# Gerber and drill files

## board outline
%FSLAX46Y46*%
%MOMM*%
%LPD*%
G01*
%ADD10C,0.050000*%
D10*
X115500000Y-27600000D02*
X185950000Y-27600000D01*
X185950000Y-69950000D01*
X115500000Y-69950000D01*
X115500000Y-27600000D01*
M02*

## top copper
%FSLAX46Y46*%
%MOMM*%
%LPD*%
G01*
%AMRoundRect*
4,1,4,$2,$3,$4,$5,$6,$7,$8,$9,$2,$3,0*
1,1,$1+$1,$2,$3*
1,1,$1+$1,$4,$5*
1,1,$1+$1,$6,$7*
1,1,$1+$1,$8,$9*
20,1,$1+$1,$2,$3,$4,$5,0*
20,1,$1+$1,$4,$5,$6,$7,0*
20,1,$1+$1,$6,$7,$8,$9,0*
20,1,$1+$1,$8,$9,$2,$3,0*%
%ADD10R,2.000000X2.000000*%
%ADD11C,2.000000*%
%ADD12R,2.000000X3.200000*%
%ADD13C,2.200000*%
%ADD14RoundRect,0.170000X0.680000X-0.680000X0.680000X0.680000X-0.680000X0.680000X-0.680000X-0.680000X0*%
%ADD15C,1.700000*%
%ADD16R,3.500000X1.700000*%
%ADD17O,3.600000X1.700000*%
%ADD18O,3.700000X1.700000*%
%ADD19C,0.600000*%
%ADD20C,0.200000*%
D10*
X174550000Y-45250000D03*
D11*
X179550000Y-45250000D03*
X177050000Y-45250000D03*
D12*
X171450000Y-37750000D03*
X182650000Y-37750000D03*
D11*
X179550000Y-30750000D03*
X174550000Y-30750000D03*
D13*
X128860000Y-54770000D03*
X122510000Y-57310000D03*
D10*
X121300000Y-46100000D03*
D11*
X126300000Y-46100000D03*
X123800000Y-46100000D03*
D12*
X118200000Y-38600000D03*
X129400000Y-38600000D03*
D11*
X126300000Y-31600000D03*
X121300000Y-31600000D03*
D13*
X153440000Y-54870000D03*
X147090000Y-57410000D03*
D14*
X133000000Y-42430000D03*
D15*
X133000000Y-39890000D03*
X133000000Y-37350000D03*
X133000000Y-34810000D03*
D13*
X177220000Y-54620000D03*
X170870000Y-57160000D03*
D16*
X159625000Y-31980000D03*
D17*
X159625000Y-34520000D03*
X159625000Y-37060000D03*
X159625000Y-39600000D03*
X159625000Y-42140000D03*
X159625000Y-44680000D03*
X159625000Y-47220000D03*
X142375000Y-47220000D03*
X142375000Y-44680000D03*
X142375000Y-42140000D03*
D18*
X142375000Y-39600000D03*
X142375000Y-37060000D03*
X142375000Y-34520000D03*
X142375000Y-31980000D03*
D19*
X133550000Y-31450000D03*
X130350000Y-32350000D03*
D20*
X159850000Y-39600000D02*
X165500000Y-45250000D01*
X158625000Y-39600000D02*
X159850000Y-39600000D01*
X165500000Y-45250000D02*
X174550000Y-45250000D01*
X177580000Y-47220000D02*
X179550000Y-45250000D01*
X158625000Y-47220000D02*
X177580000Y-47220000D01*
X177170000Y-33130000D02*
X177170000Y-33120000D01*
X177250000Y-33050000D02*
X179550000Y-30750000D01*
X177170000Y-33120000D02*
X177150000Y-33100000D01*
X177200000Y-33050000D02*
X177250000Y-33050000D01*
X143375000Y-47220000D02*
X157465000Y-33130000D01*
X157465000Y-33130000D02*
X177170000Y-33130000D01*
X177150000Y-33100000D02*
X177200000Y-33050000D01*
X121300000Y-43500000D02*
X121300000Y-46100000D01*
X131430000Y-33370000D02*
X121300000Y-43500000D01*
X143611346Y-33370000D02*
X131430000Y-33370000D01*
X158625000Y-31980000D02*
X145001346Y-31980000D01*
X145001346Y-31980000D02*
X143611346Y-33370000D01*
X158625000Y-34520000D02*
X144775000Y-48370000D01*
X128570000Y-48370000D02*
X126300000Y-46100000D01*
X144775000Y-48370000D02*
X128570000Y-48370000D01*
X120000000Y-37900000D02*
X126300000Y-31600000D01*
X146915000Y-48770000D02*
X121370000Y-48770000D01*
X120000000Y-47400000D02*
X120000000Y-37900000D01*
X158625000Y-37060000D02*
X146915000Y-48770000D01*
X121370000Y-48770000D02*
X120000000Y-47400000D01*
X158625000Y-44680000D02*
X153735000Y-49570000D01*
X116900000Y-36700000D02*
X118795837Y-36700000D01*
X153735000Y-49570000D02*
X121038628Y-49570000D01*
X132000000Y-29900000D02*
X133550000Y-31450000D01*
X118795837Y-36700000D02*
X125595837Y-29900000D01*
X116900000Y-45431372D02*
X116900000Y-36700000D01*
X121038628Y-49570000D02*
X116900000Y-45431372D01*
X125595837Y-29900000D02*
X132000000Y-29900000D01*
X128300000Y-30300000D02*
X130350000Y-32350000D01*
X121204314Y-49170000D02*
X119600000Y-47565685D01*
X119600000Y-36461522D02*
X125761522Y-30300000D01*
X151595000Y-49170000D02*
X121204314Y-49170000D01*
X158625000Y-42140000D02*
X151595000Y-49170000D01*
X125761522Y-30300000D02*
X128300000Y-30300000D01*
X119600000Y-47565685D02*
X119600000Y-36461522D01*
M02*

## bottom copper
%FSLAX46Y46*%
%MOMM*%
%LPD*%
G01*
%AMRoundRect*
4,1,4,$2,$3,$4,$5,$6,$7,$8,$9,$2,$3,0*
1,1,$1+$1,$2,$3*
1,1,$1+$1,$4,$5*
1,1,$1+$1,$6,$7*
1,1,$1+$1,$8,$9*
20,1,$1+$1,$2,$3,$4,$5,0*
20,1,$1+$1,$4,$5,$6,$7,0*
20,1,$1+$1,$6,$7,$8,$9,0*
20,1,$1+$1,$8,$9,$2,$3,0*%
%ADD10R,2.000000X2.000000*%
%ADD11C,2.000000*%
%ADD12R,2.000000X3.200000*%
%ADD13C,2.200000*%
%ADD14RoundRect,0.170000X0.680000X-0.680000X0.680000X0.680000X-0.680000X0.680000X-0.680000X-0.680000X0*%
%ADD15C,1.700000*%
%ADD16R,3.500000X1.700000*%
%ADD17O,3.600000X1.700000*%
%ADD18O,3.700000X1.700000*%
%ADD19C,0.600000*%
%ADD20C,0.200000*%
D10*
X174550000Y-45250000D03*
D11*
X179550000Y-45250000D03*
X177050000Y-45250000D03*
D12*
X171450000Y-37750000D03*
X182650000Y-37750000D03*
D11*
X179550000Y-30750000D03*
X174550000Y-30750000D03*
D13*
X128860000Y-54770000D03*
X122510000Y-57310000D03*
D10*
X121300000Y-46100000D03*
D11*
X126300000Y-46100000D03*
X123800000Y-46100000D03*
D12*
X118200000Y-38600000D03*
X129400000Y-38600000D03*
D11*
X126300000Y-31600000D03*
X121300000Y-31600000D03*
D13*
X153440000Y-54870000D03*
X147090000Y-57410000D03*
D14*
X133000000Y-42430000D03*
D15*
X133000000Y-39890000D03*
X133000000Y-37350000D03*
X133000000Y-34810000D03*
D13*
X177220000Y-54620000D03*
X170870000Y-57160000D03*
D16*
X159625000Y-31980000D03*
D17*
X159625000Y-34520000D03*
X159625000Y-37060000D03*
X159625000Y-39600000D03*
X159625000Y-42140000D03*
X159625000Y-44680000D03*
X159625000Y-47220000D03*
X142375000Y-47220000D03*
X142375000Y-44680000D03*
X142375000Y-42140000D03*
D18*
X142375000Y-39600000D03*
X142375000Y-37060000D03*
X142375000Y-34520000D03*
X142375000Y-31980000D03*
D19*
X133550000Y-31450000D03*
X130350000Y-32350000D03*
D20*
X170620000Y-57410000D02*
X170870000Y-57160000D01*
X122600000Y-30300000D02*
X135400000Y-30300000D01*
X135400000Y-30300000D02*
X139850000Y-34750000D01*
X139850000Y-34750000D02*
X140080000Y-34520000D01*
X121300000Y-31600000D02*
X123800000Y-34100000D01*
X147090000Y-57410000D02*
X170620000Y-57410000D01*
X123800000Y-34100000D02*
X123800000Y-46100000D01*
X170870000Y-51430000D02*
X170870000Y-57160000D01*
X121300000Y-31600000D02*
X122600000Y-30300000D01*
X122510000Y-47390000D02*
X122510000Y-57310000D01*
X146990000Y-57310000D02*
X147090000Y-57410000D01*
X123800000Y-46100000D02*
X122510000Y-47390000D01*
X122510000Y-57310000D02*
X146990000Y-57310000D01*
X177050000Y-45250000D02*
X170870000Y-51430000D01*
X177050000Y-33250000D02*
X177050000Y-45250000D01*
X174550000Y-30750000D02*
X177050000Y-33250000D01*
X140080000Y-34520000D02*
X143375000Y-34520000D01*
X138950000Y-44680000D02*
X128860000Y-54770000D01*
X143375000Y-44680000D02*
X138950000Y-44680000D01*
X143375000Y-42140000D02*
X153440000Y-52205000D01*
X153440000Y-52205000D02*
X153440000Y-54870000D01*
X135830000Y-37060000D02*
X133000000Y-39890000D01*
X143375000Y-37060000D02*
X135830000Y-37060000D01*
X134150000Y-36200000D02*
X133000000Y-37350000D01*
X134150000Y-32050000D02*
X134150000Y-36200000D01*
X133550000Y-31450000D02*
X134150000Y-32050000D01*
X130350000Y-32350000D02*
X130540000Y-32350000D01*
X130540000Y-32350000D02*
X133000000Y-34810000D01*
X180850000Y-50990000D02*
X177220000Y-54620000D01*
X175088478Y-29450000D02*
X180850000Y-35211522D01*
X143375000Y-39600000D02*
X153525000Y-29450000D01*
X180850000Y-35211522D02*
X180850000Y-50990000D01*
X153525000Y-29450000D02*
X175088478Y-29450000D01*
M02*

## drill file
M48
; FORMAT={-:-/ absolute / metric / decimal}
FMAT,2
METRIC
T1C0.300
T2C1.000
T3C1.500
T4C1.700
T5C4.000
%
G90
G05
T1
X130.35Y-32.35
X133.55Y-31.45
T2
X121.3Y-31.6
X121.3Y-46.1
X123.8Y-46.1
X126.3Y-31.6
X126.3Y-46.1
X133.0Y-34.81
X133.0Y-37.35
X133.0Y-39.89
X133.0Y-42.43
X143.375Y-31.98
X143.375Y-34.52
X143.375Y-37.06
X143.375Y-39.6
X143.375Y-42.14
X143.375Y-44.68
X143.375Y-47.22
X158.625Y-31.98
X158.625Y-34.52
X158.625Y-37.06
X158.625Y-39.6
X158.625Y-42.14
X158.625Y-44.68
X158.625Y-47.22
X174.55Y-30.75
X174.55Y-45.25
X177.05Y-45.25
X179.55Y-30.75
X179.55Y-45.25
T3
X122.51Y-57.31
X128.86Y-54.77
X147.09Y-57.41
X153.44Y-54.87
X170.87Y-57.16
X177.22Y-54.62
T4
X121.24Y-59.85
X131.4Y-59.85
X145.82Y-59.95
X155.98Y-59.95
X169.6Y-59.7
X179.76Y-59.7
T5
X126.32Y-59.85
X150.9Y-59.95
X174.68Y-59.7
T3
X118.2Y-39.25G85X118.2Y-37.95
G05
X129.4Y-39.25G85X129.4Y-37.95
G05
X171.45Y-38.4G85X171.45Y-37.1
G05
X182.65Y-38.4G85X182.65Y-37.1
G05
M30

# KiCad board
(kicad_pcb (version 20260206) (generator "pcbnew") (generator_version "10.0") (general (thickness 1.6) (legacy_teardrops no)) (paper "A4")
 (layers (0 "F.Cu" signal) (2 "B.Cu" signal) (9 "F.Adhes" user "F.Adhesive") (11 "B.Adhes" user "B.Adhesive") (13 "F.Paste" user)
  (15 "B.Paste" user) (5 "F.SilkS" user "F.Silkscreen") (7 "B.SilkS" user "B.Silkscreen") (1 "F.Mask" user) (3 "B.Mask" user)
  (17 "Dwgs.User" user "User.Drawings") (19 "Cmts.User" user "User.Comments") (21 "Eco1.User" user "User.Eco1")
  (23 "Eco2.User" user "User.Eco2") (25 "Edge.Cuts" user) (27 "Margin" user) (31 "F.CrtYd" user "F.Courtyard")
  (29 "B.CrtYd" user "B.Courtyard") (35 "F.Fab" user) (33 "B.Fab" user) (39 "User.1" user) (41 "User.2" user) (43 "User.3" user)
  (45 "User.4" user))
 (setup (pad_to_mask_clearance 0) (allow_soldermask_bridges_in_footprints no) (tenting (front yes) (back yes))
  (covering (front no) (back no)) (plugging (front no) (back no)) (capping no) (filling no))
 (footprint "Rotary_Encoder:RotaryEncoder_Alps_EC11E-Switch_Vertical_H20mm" (layer "F.Cu") (at 174.55 45.25 90)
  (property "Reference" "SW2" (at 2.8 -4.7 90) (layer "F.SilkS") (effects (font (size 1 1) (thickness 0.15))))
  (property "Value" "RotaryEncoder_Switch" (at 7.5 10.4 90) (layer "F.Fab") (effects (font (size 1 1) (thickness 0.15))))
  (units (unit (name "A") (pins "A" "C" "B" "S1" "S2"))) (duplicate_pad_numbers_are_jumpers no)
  (pad "A" thru_hole rect (at 0 0 90) (size 2 2) (drill 1) (layers "*.Cu" "*.Mask") (remove_unused_layers no) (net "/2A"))
  (pad "B" thru_hole circle (at 0 5 90) (size 2 2) (drill 1) (layers "*.Cu" "*.Mask") (remove_unused_layers no) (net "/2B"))
  (pad "C" thru_hole circle (at 0 2.5 90) (size 2 2) (drill 1) (layers "*.Cu" "*.Mask") (remove_unused_layers no) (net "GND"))
  (pad "MP" thru_hole rect (at 7.5 -3.1 90) (size 3.2 2) (drill oval 2.8 1.5) (layers "*.Cu" "*.Mask") (remove_unused_layers no))
  (pad "MP" thru_hole rect (at 7.5 8.1 90) (size 3.2 2) (drill oval 2.8 1.5) (layers "*.Cu" "*.Mask") (remove_unused_layers no))
  (pad "S1" thru_hole circle (at 14.5 5 90) (size 2 2) (drill 1) (layers "*.Cu" "*.Mask") (remove_unused_layers no) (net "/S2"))
  (pad "S2" thru_hole circle (at 14.5 0 90) (size 2 2) (drill 1) (layers "*.Cu" "*.Mask") (remove_unused_layers no) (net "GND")))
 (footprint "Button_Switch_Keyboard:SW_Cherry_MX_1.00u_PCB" (layer "F.Cu") (at 128.86 54.77)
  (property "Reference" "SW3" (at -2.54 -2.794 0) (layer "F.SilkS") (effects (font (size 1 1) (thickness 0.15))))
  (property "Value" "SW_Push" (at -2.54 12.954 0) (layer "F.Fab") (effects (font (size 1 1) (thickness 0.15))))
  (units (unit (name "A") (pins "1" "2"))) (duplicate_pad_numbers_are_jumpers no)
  (pad "" np_thru_hole circle (at -7.62 5.08) (size 1.7 1.7) (drill 1.7) (layers "*.Cu" "*.Mask"))
  (pad "" np_thru_hole circle (at -2.54 5.08) (size 4 4) (drill 4) (layers "*.Cu" "*.Mask"))
  (pad "" np_thru_hole circle (at 2.54 5.08) (size 1.7 1.7) (drill 1.7) (layers "*.Cu" "*.Mask"))
  (pad "1" thru_hole circle (at 0 0) (size 2.2 2.2) (drill 1.5) (layers "*.Cu" "*.Mask") (remove_unused_layers no) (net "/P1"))
  (pad "2" thru_hole circle (at -6.35 2.54) (size 2.2 2.2) (drill 1.5) (layers "*.Cu" "*.Mask") (remove_unused_layers no) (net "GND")))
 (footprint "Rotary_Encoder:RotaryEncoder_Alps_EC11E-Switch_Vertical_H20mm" (layer "F.Cu") (at 121.3 46.1 90)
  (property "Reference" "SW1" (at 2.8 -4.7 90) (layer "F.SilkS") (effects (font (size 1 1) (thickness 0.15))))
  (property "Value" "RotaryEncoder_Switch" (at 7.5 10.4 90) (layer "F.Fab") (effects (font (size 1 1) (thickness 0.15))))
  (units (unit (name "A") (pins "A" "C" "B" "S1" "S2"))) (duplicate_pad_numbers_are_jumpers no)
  (pad "A" thru_hole rect (at 0 0 90) (size 2 2) (drill 1) (layers "*.Cu" "*.Mask") (remove_unused_layers no) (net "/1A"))
  (pad "B" thru_hole circle (at 0 5 90) (size 2 2) (drill 1) (layers "*.Cu" "*.Mask") (remove_unused_layers no) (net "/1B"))
  (pad "C" thru_hole circle (at 0 2.5 90) (size 2 2) (drill 1) (layers "*.Cu" "*.Mask") (remove_unused_layers no) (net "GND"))
  (pad "MP" thru_hole rect (at 7.5 -3.1 90) (size 3.2 2) (drill oval 2.8 1.5) (layers "*.Cu" "*.Mask") (remove_unused_layers no))
  (pad "MP" thru_hole rect (at 7.5 8.1 90) (size 3.2 2) (drill oval 2.8 1.5) (layers "*.Cu" "*.Mask") (remove_unused_layers no))
  (pad "S1" thru_hole circle (at 14.5 5 90) (size 2 2) (drill 1) (layers "*.Cu" "*.Mask") (remove_unused_layers no) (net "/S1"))
  (pad "S2" thru_hole circle (at 14.5 0 90) (size 2 2) (drill 1) (layers "*.Cu" "*.Mask") (remove_unused_layers no) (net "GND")))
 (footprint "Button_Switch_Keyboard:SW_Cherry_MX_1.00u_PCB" (layer "F.Cu") (at 153.44 54.87)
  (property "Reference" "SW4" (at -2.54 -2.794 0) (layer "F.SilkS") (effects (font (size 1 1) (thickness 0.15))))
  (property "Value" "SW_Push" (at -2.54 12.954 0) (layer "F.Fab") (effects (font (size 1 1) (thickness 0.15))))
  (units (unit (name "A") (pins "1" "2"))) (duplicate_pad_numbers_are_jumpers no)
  (pad "" np_thru_hole circle (at -7.62 5.08) (size 1.7 1.7) (drill 1.7) (layers "*.Cu" "*.Mask"))
  (pad "" np_thru_hole circle (at -2.54 5.08) (size 4 4) (drill 4) (layers "*.Cu" "*.Mask"))
  (pad "" np_thru_hole circle (at 2.54 5.08) (size 1.7 1.7) (drill 1.7) (layers "*.Cu" "*.Mask"))
  (pad "1" thru_hole circle (at 0 0) (size 2.2 2.2) (drill 1.5) (layers "*.Cu" "*.Mask") (remove_unused_layers no) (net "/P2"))
  (pad "2" thru_hole circle (at -6.35 2.54) (size 2.2 2.2) (drill 1.5) (layers "*.Cu" "*.Mask") (remove_unused_layers no) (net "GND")))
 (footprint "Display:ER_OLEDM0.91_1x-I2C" (layer "F.Cu") (at 133 42.43 90)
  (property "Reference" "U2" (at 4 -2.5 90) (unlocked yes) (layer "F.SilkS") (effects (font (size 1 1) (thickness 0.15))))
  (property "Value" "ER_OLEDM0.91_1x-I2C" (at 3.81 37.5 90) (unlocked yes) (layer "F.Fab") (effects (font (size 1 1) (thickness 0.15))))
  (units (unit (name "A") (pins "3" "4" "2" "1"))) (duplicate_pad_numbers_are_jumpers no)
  (pad "1" thru_hole roundrect (at 0 0 90) (size 1.7 1.7) (drill 1) (layers "*.Cu" "*.Mask") (remove_unused_layers no)
   (roundrect_rratio 0.1) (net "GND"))
  (pad "2" thru_hole circle (at 2.54 0 90) (size 1.7 1.7) (drill 1) (layers "*.Cu" "*.Mask") (remove_unused_layers no) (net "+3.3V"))
  (pad "3" thru_hole circle (at 5.08 0 90) (size 1.7 1.7) (drill 1) (layers "*.Cu" "*.Mask") (remove_unused_layers no) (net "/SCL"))
  (pad "4" thru_hole circle (at 7.62 0 90) (size 1.7 1.7) (drill 1) (layers "*.Cu" "*.Mask") (remove_unused_layers no) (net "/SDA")))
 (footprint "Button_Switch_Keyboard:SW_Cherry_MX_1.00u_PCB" (layer "F.Cu") (at 177.22 54.62)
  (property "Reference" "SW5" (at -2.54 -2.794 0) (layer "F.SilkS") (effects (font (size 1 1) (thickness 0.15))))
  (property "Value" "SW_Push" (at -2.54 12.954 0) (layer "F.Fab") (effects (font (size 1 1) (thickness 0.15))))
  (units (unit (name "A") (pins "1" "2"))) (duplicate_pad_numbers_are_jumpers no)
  (pad "" np_thru_hole circle (at -7.62 5.08) (size 1.7 1.7) (drill 1.7) (layers "*.Cu" "*.Mask"))
  (pad "" np_thru_hole circle (at -2.54 5.08) (size 4 4) (drill 4) (layers "*.Cu" "*.Mask"))
  (pad "" np_thru_hole circle (at 2.54 5.08) (size 1.7 1.7) (drill 1.7) (layers "*.Cu" "*.Mask"))
  (pad "1" thru_hole circle (at 0 0) (size 2.2 2.2) (drill 1.5) (layers "*.Cu" "*.Mask") (remove_unused_layers no) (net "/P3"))
  (pad "2" thru_hole circle (at -6.35 2.54) (size 2.2 2.2) (drill 1.5) (layers "*.Cu" "*.Mask") (remove_unused_layers no) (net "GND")))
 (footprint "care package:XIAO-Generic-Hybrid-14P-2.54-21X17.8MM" (layer "B.Cu") (at 151 39.6 180)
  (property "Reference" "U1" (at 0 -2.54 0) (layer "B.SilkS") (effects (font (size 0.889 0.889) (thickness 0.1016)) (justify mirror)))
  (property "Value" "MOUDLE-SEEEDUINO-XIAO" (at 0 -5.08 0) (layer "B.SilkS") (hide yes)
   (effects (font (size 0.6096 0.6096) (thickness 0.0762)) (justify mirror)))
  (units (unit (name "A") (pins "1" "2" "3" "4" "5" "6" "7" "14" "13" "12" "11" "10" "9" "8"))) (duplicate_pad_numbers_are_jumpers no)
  (pad "1" thru_hole rect (at -7.625 7.62 180) (size 3.5 1.7) (drill 1 (offset -1 0)) (layers "*.Cu" "*.Mask") (remove_unused_layers no)
   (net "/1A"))
  (pad "2" thru_hole oval (at -7.625 5.08 180) (size 3.6 1.7) (drill 1 (offset -1 0)) (layers "*.Cu" "*.Mask") (remove_unused_layers no)
   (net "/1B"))
  (pad "3" thru_hole oval (at -7.625 2.54 180) (size 3.6 1.7) (drill 1 (offset -1 0)) (layers "*.Cu" "*.Mask") (remove_unused_layers no)
   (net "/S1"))
  (pad "4" thru_hole oval (at -7.625 0 180) (size 3.6 1.7) (drill 1 (offset -1 0)) (layers "*.Cu" "*.Mask") (remove_unused_layers no)
   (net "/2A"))
  (pad "5" thru_hole oval (at -7.625 -2.54 180) (size 3.6 1.7) (drill 1 (offset -1 0)) (layers "*.Cu" "*.Mask") (remove_unused_layers no)
   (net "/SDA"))
  (pad "6" thru_hole oval (at -7.625 -5.08) (size 3.6 1.7) (drill 1 (offset 1 0)) (layers "*.Cu" "*.Mask") (remove_unused_layers no)
   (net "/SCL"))
  (pad "7" thru_hole oval (at -7.625 -7.62 180) (size 3.6 1.7) (drill 1 (offset -1 0)) (layers "*.Cu" "*.Mask") (remove_unused_layers no)
   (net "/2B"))
  (pad "8" thru_hole oval (at 7.625 -7.62 180) (size 3.6 1.7) (drill 1 (offset 1 0)) (layers "*.Cu" "*.Mask") (remove_unused_layers no)
   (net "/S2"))
  (pad "9" thru_hole oval (at 7.625 -5.08 180) (size 3.6 1.7) (drill 1 (offset 1 0)) (layers "*.Cu" "*.Mask") (remove_unused_layers no)
   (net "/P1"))
  (pad "10" thru_hole oval (at 7.625 -2.54 180) (size 3.6 1.7) (drill 1 (offset 1 0)) (layers "*.Cu" "*.Mask") (remove_unused_layers no)
   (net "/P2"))
  (pad "11" thru_hole oval (at 7.625 0 180) (size 3.7 1.7) (drill 1 (offset 1 0)) (layers "*.Cu" "*.Mask") (remove_unused_layers no)
   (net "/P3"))
  (pad "12" thru_hole oval (at 7.625 2.54 180) (size 3.7 1.7) (drill 1 (offset 1 0)) (layers "*.Cu" "*.Mask") (remove_unused_layers no)
   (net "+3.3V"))
  (pad "13" thru_hole oval (at 7.625 5.08 180) (size 3.7 1.7) (drill 1 (offset 1 0)) (layers "*.Cu" "*.Mask") (remove_unused_layers no)
   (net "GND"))
  (pad "14" thru_hole oval (at 7.625 7.62 180) (size 3.7 1.7) (drill 1 (offset 1 0)) (layers "*.Cu" "*.Mask") (remove_unused_layers no)
   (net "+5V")))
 (gr_rect (start 115.5 27.6) (end 185.95 69.95) (stroke (width 0.05) (type default)) (fill no) (layer "Edge.Cuts"))
 (segment (start 159.85 39.6) (end 165.5 45.25) (width 0.2) (layer "F.Cu") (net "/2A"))
 (segment (start 158.625 39.6) (end 159.85 39.6) (width 0.2) (layer "F.Cu") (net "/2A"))
 (segment (start 165.5 45.25) (end 174.55 45.25) (width 0.2) (layer "F.Cu") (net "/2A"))
 (segment (start 177.58 47.22) (end 179.55 45.25) (width 0.2) (layer "F.Cu") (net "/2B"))
 (segment (start 158.625 47.22) (end 177.58 47.22) (width 0.2) (layer "F.Cu") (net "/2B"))
 (segment (start 170.62 57.41) (end 170.87 57.16) (width 0.2) (layer "B.Cu") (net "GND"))
 (segment (start 122.6 30.3) (end 135.4 30.3) (width 0.2) (layer "B.Cu") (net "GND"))
 (segment (start 135.4 30.3) (end 139.85 34.75) (width 0.2) (layer "B.Cu") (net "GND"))
 (segment (start 139.85 34.75) (end 140.08 34.52) (width 0.2) (layer "B.Cu") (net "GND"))
 (segment (start 121.3 31.6) (end 123.8 34.1) (width 0.2) (layer "B.Cu") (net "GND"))
 (segment (start 147.09 57.41) (end 170.62 57.41) (width 0.2) (layer "B.Cu") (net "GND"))
 (segment (start 123.8 34.1) (end 123.8 46.1) (width 0.2) (layer "B.Cu") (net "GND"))
 (segment (start 170.87 51.43) (end 170.87 57.16) (width 0.2) (layer "B.Cu") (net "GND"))
 (segment (start 121.3 31.6) (end 122.6 30.3) (width 0.2) (layer "B.Cu") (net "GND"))
 (segment (start 122.51 47.39) (end 122.51 57.31) (width 0.2) (layer "B.Cu") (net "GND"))
 (segment (start 146.99 57.31) (end 147.09 57.41) (width 0.2) (layer "B.Cu") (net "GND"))
 (segment (start 123.8 46.1) (end 122.51 47.39) (width 0.2) (layer "B.Cu") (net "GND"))
 (segment (start 122.51 57.31) (end 146.99 57.31) (width 0.2) (layer "B.Cu") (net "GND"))
 (segment (start 177.05 45.25) (end 170.87 51.43) (width 0.2) (layer "B.Cu") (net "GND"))
 (segment (start 177.05 33.25) (end 177.05 45.25) (width 0.2) (layer "B.Cu") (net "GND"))
 (segment (start 174.55 30.75) (end 177.05 33.25) (width 0.2) (layer "B.Cu") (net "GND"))
 (segment (start 140.08 34.52) (end 143.375 34.52) (width 0.2) (layer "B.Cu") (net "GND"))
 (segment (start 177.17 33.13) (end 177.17 33.12) (width 0.2) (layer "F.Cu") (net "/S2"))
 (segment (start 177.25 33.05) (end 179.55 30.75) (width 0.2) (layer "F.Cu") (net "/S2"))
 (segment (start 177.17 33.12) (end 177.15 33.1) (width 0.2) (layer "F.Cu") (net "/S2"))
 (segment (start 177.2 33.05) (end 177.25 33.05) (width 0.2) (layer "F.Cu") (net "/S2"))
 (segment (start 143.375 47.22) (end 157.465 33.13) (width 0.2) (layer "F.Cu") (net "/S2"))
 (segment (start 157.465 33.13) (end 177.17 33.13) (width 0.2) (layer "F.Cu") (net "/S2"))
 (segment (start 177.15 33.1) (end 177.2 33.05) (width 0.2) (layer "F.Cu") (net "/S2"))
 (segment (start 138.95 44.68) (end 128.86 54.77) (width 0.2) (layer "B.Cu") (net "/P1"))
 (segment (start 143.375 44.68) (end 138.95 44.68) (width 0.2) (layer "B.Cu") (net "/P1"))
 (segment (start 121.3 43.5) (end 121.3 46.1) (width 0.2) (layer "F.Cu") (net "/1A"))
 (segment (start 131.43 33.37) (end 121.3 43.5) (width 0.2) (layer "F.Cu") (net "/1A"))
 (segment (start 143.611346 33.37) (end 131.43 33.37) (width 0.2) (layer "F.Cu") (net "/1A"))
 (segment (start 158.625 31.98) (end 145.001346 31.98) (width 0.2) (layer "F.Cu") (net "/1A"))
 (segment (start 145.001346 31.98) (end 143.611346 33.37) (width 0.2) (layer "F.Cu") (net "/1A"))
 (segment (start 158.625 34.52) (end 144.775 48.37) (width 0.2) (layer "F.Cu") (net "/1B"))
 (segment (start 128.57 48.37) (end 126.3 46.1) (width 0.2) (layer "F.Cu") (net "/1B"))
 (segment (start 144.775 48.37) (end 128.57 48.37) (width 0.2) (layer "F.Cu") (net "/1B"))
 (segment (start 120 37.9) (end 126.3 31.6) (width 0.2) (layer "F.Cu") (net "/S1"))
 (segment (start 146.915 48.77) (end 121.37 48.77) (width 0.2) (layer "F.Cu") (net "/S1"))
 (segment (start 120 47.4) (end 120 37.9) (width 0.2) (layer "F.Cu") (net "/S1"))
 (segment (start 158.625 37.06) (end 146.915 48.77) (width 0.2) (layer "F.Cu") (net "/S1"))
 (segment (start 121.37 48.77) (end 120 47.4) (width 0.2) (layer "F.Cu") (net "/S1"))
 (segment (start 143.375 42.14) (end 153.44 52.205) (width 0.2) (layer "B.Cu") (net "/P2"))
 (segment (start 153.44 52.205) (end 153.44 54.87) (width 0.2) (layer "B.Cu") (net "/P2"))
 (segment (start 135.83 37.06) (end 133 39.89) (width 0.2) (layer "B.Cu") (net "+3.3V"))
 (segment (start 143.375 37.06) (end 135.83 37.06) (width 0.2) (layer "B.Cu") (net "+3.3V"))
 (segment (start 158.625 44.68) (end 153.735 49.57) (width 0.2) (layer "F.Cu") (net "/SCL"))
 (segment (start 116.9 36.7) (end 118.795837 36.7) (width 0.2) (layer "F.Cu") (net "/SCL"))
 (segment (start 153.735 49.57) (end 121.038628 49.57) (width 0.2) (layer "F.Cu") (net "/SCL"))
 (segment (start 132 29.9) (end 133.55 31.45) (width 0.2) (layer "F.Cu") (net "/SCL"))
 (segment (start 118.795837 36.7) (end 125.595837 29.9) (width 0.2) (layer "F.Cu") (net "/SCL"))
 (segment (start 116.9 45.431372) (end 116.9 36.7) (width 0.2) (layer "F.Cu") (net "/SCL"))
 (segment (start 121.038628 49.57) (end 116.9 45.431372) (width 0.2) (layer "F.Cu") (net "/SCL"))
 (segment (start 125.595837 29.9) (end 132 29.9) (width 0.2) (layer "F.Cu") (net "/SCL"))
 (via (at 133.55 31.45) (size 0.6) (drill 0.3) (layers "F.Cu" "B.Cu") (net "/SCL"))
 (segment (start 134.15 36.2) (end 133 37.35) (width 0.2) (layer "B.Cu") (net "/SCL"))
 (segment (start 134.15 32.05) (end 134.15 36.2) (width 0.2) (layer "B.Cu") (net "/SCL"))
 (segment (start 133.55 31.45) (end 134.15 32.05) (width 0.2) (layer "B.Cu") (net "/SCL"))
 (segment (start 128.3 30.3) (end 130.35 32.35) (width 0.2) (layer "F.Cu") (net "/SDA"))
 (segment (start 121.204314 49.17) (end 119.6 47.565685) (width 0.2) (layer "F.Cu") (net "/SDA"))
 (segment (start 119.6 36.461522) (end 125.761522 30.3) (width 0.2) (layer "F.Cu") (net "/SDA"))
 (segment (start 151.595 49.17) (end 121.204314 49.17) (width 0.2) (layer "F.Cu") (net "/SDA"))
 (segment (start 158.625 42.14) (end 151.595 49.17) (width 0.2) (layer "F.Cu") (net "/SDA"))
 (segment (start 125.761522 30.3) (end 128.3 30.3) (width 0.2) (layer "F.Cu") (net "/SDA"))
 (segment (start 119.6 47.565685) (end 119.6 36.461522) (width 0.2) (layer "F.Cu") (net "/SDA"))
 (via (at 130.35 32.35) (size 0.6) (drill 0.3) (layers "F.Cu" "B.Cu") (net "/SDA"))
 (segment (start 130.35 32.35) (end 130.54 32.35) (width 0.2) (layer "B.Cu") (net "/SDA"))
 (segment (start 130.54 32.35) (end 133 34.81) (width 0.2) (layer "B.Cu") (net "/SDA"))
 (segment (start 180.85 50.99) (end 177.22 54.62) (width 0.2) (layer "B.Cu") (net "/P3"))
 (segment (start 175.088478 29.45) (end 180.85 35.211522) (width 0.2) (layer "B.Cu") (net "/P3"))
 (segment (start 143.375 39.6) (end 153.525 29.45) (width 0.2) (layer "B.Cu") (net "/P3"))
 (segment (start 180.85 35.211522) (end 180.85 50.99) (width 0.2) (layer "B.Cu") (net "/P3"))
 (segment (start 153.525 29.45) (end 175.088478 29.45) (width 0.2) (layer "B.Cu") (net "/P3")))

